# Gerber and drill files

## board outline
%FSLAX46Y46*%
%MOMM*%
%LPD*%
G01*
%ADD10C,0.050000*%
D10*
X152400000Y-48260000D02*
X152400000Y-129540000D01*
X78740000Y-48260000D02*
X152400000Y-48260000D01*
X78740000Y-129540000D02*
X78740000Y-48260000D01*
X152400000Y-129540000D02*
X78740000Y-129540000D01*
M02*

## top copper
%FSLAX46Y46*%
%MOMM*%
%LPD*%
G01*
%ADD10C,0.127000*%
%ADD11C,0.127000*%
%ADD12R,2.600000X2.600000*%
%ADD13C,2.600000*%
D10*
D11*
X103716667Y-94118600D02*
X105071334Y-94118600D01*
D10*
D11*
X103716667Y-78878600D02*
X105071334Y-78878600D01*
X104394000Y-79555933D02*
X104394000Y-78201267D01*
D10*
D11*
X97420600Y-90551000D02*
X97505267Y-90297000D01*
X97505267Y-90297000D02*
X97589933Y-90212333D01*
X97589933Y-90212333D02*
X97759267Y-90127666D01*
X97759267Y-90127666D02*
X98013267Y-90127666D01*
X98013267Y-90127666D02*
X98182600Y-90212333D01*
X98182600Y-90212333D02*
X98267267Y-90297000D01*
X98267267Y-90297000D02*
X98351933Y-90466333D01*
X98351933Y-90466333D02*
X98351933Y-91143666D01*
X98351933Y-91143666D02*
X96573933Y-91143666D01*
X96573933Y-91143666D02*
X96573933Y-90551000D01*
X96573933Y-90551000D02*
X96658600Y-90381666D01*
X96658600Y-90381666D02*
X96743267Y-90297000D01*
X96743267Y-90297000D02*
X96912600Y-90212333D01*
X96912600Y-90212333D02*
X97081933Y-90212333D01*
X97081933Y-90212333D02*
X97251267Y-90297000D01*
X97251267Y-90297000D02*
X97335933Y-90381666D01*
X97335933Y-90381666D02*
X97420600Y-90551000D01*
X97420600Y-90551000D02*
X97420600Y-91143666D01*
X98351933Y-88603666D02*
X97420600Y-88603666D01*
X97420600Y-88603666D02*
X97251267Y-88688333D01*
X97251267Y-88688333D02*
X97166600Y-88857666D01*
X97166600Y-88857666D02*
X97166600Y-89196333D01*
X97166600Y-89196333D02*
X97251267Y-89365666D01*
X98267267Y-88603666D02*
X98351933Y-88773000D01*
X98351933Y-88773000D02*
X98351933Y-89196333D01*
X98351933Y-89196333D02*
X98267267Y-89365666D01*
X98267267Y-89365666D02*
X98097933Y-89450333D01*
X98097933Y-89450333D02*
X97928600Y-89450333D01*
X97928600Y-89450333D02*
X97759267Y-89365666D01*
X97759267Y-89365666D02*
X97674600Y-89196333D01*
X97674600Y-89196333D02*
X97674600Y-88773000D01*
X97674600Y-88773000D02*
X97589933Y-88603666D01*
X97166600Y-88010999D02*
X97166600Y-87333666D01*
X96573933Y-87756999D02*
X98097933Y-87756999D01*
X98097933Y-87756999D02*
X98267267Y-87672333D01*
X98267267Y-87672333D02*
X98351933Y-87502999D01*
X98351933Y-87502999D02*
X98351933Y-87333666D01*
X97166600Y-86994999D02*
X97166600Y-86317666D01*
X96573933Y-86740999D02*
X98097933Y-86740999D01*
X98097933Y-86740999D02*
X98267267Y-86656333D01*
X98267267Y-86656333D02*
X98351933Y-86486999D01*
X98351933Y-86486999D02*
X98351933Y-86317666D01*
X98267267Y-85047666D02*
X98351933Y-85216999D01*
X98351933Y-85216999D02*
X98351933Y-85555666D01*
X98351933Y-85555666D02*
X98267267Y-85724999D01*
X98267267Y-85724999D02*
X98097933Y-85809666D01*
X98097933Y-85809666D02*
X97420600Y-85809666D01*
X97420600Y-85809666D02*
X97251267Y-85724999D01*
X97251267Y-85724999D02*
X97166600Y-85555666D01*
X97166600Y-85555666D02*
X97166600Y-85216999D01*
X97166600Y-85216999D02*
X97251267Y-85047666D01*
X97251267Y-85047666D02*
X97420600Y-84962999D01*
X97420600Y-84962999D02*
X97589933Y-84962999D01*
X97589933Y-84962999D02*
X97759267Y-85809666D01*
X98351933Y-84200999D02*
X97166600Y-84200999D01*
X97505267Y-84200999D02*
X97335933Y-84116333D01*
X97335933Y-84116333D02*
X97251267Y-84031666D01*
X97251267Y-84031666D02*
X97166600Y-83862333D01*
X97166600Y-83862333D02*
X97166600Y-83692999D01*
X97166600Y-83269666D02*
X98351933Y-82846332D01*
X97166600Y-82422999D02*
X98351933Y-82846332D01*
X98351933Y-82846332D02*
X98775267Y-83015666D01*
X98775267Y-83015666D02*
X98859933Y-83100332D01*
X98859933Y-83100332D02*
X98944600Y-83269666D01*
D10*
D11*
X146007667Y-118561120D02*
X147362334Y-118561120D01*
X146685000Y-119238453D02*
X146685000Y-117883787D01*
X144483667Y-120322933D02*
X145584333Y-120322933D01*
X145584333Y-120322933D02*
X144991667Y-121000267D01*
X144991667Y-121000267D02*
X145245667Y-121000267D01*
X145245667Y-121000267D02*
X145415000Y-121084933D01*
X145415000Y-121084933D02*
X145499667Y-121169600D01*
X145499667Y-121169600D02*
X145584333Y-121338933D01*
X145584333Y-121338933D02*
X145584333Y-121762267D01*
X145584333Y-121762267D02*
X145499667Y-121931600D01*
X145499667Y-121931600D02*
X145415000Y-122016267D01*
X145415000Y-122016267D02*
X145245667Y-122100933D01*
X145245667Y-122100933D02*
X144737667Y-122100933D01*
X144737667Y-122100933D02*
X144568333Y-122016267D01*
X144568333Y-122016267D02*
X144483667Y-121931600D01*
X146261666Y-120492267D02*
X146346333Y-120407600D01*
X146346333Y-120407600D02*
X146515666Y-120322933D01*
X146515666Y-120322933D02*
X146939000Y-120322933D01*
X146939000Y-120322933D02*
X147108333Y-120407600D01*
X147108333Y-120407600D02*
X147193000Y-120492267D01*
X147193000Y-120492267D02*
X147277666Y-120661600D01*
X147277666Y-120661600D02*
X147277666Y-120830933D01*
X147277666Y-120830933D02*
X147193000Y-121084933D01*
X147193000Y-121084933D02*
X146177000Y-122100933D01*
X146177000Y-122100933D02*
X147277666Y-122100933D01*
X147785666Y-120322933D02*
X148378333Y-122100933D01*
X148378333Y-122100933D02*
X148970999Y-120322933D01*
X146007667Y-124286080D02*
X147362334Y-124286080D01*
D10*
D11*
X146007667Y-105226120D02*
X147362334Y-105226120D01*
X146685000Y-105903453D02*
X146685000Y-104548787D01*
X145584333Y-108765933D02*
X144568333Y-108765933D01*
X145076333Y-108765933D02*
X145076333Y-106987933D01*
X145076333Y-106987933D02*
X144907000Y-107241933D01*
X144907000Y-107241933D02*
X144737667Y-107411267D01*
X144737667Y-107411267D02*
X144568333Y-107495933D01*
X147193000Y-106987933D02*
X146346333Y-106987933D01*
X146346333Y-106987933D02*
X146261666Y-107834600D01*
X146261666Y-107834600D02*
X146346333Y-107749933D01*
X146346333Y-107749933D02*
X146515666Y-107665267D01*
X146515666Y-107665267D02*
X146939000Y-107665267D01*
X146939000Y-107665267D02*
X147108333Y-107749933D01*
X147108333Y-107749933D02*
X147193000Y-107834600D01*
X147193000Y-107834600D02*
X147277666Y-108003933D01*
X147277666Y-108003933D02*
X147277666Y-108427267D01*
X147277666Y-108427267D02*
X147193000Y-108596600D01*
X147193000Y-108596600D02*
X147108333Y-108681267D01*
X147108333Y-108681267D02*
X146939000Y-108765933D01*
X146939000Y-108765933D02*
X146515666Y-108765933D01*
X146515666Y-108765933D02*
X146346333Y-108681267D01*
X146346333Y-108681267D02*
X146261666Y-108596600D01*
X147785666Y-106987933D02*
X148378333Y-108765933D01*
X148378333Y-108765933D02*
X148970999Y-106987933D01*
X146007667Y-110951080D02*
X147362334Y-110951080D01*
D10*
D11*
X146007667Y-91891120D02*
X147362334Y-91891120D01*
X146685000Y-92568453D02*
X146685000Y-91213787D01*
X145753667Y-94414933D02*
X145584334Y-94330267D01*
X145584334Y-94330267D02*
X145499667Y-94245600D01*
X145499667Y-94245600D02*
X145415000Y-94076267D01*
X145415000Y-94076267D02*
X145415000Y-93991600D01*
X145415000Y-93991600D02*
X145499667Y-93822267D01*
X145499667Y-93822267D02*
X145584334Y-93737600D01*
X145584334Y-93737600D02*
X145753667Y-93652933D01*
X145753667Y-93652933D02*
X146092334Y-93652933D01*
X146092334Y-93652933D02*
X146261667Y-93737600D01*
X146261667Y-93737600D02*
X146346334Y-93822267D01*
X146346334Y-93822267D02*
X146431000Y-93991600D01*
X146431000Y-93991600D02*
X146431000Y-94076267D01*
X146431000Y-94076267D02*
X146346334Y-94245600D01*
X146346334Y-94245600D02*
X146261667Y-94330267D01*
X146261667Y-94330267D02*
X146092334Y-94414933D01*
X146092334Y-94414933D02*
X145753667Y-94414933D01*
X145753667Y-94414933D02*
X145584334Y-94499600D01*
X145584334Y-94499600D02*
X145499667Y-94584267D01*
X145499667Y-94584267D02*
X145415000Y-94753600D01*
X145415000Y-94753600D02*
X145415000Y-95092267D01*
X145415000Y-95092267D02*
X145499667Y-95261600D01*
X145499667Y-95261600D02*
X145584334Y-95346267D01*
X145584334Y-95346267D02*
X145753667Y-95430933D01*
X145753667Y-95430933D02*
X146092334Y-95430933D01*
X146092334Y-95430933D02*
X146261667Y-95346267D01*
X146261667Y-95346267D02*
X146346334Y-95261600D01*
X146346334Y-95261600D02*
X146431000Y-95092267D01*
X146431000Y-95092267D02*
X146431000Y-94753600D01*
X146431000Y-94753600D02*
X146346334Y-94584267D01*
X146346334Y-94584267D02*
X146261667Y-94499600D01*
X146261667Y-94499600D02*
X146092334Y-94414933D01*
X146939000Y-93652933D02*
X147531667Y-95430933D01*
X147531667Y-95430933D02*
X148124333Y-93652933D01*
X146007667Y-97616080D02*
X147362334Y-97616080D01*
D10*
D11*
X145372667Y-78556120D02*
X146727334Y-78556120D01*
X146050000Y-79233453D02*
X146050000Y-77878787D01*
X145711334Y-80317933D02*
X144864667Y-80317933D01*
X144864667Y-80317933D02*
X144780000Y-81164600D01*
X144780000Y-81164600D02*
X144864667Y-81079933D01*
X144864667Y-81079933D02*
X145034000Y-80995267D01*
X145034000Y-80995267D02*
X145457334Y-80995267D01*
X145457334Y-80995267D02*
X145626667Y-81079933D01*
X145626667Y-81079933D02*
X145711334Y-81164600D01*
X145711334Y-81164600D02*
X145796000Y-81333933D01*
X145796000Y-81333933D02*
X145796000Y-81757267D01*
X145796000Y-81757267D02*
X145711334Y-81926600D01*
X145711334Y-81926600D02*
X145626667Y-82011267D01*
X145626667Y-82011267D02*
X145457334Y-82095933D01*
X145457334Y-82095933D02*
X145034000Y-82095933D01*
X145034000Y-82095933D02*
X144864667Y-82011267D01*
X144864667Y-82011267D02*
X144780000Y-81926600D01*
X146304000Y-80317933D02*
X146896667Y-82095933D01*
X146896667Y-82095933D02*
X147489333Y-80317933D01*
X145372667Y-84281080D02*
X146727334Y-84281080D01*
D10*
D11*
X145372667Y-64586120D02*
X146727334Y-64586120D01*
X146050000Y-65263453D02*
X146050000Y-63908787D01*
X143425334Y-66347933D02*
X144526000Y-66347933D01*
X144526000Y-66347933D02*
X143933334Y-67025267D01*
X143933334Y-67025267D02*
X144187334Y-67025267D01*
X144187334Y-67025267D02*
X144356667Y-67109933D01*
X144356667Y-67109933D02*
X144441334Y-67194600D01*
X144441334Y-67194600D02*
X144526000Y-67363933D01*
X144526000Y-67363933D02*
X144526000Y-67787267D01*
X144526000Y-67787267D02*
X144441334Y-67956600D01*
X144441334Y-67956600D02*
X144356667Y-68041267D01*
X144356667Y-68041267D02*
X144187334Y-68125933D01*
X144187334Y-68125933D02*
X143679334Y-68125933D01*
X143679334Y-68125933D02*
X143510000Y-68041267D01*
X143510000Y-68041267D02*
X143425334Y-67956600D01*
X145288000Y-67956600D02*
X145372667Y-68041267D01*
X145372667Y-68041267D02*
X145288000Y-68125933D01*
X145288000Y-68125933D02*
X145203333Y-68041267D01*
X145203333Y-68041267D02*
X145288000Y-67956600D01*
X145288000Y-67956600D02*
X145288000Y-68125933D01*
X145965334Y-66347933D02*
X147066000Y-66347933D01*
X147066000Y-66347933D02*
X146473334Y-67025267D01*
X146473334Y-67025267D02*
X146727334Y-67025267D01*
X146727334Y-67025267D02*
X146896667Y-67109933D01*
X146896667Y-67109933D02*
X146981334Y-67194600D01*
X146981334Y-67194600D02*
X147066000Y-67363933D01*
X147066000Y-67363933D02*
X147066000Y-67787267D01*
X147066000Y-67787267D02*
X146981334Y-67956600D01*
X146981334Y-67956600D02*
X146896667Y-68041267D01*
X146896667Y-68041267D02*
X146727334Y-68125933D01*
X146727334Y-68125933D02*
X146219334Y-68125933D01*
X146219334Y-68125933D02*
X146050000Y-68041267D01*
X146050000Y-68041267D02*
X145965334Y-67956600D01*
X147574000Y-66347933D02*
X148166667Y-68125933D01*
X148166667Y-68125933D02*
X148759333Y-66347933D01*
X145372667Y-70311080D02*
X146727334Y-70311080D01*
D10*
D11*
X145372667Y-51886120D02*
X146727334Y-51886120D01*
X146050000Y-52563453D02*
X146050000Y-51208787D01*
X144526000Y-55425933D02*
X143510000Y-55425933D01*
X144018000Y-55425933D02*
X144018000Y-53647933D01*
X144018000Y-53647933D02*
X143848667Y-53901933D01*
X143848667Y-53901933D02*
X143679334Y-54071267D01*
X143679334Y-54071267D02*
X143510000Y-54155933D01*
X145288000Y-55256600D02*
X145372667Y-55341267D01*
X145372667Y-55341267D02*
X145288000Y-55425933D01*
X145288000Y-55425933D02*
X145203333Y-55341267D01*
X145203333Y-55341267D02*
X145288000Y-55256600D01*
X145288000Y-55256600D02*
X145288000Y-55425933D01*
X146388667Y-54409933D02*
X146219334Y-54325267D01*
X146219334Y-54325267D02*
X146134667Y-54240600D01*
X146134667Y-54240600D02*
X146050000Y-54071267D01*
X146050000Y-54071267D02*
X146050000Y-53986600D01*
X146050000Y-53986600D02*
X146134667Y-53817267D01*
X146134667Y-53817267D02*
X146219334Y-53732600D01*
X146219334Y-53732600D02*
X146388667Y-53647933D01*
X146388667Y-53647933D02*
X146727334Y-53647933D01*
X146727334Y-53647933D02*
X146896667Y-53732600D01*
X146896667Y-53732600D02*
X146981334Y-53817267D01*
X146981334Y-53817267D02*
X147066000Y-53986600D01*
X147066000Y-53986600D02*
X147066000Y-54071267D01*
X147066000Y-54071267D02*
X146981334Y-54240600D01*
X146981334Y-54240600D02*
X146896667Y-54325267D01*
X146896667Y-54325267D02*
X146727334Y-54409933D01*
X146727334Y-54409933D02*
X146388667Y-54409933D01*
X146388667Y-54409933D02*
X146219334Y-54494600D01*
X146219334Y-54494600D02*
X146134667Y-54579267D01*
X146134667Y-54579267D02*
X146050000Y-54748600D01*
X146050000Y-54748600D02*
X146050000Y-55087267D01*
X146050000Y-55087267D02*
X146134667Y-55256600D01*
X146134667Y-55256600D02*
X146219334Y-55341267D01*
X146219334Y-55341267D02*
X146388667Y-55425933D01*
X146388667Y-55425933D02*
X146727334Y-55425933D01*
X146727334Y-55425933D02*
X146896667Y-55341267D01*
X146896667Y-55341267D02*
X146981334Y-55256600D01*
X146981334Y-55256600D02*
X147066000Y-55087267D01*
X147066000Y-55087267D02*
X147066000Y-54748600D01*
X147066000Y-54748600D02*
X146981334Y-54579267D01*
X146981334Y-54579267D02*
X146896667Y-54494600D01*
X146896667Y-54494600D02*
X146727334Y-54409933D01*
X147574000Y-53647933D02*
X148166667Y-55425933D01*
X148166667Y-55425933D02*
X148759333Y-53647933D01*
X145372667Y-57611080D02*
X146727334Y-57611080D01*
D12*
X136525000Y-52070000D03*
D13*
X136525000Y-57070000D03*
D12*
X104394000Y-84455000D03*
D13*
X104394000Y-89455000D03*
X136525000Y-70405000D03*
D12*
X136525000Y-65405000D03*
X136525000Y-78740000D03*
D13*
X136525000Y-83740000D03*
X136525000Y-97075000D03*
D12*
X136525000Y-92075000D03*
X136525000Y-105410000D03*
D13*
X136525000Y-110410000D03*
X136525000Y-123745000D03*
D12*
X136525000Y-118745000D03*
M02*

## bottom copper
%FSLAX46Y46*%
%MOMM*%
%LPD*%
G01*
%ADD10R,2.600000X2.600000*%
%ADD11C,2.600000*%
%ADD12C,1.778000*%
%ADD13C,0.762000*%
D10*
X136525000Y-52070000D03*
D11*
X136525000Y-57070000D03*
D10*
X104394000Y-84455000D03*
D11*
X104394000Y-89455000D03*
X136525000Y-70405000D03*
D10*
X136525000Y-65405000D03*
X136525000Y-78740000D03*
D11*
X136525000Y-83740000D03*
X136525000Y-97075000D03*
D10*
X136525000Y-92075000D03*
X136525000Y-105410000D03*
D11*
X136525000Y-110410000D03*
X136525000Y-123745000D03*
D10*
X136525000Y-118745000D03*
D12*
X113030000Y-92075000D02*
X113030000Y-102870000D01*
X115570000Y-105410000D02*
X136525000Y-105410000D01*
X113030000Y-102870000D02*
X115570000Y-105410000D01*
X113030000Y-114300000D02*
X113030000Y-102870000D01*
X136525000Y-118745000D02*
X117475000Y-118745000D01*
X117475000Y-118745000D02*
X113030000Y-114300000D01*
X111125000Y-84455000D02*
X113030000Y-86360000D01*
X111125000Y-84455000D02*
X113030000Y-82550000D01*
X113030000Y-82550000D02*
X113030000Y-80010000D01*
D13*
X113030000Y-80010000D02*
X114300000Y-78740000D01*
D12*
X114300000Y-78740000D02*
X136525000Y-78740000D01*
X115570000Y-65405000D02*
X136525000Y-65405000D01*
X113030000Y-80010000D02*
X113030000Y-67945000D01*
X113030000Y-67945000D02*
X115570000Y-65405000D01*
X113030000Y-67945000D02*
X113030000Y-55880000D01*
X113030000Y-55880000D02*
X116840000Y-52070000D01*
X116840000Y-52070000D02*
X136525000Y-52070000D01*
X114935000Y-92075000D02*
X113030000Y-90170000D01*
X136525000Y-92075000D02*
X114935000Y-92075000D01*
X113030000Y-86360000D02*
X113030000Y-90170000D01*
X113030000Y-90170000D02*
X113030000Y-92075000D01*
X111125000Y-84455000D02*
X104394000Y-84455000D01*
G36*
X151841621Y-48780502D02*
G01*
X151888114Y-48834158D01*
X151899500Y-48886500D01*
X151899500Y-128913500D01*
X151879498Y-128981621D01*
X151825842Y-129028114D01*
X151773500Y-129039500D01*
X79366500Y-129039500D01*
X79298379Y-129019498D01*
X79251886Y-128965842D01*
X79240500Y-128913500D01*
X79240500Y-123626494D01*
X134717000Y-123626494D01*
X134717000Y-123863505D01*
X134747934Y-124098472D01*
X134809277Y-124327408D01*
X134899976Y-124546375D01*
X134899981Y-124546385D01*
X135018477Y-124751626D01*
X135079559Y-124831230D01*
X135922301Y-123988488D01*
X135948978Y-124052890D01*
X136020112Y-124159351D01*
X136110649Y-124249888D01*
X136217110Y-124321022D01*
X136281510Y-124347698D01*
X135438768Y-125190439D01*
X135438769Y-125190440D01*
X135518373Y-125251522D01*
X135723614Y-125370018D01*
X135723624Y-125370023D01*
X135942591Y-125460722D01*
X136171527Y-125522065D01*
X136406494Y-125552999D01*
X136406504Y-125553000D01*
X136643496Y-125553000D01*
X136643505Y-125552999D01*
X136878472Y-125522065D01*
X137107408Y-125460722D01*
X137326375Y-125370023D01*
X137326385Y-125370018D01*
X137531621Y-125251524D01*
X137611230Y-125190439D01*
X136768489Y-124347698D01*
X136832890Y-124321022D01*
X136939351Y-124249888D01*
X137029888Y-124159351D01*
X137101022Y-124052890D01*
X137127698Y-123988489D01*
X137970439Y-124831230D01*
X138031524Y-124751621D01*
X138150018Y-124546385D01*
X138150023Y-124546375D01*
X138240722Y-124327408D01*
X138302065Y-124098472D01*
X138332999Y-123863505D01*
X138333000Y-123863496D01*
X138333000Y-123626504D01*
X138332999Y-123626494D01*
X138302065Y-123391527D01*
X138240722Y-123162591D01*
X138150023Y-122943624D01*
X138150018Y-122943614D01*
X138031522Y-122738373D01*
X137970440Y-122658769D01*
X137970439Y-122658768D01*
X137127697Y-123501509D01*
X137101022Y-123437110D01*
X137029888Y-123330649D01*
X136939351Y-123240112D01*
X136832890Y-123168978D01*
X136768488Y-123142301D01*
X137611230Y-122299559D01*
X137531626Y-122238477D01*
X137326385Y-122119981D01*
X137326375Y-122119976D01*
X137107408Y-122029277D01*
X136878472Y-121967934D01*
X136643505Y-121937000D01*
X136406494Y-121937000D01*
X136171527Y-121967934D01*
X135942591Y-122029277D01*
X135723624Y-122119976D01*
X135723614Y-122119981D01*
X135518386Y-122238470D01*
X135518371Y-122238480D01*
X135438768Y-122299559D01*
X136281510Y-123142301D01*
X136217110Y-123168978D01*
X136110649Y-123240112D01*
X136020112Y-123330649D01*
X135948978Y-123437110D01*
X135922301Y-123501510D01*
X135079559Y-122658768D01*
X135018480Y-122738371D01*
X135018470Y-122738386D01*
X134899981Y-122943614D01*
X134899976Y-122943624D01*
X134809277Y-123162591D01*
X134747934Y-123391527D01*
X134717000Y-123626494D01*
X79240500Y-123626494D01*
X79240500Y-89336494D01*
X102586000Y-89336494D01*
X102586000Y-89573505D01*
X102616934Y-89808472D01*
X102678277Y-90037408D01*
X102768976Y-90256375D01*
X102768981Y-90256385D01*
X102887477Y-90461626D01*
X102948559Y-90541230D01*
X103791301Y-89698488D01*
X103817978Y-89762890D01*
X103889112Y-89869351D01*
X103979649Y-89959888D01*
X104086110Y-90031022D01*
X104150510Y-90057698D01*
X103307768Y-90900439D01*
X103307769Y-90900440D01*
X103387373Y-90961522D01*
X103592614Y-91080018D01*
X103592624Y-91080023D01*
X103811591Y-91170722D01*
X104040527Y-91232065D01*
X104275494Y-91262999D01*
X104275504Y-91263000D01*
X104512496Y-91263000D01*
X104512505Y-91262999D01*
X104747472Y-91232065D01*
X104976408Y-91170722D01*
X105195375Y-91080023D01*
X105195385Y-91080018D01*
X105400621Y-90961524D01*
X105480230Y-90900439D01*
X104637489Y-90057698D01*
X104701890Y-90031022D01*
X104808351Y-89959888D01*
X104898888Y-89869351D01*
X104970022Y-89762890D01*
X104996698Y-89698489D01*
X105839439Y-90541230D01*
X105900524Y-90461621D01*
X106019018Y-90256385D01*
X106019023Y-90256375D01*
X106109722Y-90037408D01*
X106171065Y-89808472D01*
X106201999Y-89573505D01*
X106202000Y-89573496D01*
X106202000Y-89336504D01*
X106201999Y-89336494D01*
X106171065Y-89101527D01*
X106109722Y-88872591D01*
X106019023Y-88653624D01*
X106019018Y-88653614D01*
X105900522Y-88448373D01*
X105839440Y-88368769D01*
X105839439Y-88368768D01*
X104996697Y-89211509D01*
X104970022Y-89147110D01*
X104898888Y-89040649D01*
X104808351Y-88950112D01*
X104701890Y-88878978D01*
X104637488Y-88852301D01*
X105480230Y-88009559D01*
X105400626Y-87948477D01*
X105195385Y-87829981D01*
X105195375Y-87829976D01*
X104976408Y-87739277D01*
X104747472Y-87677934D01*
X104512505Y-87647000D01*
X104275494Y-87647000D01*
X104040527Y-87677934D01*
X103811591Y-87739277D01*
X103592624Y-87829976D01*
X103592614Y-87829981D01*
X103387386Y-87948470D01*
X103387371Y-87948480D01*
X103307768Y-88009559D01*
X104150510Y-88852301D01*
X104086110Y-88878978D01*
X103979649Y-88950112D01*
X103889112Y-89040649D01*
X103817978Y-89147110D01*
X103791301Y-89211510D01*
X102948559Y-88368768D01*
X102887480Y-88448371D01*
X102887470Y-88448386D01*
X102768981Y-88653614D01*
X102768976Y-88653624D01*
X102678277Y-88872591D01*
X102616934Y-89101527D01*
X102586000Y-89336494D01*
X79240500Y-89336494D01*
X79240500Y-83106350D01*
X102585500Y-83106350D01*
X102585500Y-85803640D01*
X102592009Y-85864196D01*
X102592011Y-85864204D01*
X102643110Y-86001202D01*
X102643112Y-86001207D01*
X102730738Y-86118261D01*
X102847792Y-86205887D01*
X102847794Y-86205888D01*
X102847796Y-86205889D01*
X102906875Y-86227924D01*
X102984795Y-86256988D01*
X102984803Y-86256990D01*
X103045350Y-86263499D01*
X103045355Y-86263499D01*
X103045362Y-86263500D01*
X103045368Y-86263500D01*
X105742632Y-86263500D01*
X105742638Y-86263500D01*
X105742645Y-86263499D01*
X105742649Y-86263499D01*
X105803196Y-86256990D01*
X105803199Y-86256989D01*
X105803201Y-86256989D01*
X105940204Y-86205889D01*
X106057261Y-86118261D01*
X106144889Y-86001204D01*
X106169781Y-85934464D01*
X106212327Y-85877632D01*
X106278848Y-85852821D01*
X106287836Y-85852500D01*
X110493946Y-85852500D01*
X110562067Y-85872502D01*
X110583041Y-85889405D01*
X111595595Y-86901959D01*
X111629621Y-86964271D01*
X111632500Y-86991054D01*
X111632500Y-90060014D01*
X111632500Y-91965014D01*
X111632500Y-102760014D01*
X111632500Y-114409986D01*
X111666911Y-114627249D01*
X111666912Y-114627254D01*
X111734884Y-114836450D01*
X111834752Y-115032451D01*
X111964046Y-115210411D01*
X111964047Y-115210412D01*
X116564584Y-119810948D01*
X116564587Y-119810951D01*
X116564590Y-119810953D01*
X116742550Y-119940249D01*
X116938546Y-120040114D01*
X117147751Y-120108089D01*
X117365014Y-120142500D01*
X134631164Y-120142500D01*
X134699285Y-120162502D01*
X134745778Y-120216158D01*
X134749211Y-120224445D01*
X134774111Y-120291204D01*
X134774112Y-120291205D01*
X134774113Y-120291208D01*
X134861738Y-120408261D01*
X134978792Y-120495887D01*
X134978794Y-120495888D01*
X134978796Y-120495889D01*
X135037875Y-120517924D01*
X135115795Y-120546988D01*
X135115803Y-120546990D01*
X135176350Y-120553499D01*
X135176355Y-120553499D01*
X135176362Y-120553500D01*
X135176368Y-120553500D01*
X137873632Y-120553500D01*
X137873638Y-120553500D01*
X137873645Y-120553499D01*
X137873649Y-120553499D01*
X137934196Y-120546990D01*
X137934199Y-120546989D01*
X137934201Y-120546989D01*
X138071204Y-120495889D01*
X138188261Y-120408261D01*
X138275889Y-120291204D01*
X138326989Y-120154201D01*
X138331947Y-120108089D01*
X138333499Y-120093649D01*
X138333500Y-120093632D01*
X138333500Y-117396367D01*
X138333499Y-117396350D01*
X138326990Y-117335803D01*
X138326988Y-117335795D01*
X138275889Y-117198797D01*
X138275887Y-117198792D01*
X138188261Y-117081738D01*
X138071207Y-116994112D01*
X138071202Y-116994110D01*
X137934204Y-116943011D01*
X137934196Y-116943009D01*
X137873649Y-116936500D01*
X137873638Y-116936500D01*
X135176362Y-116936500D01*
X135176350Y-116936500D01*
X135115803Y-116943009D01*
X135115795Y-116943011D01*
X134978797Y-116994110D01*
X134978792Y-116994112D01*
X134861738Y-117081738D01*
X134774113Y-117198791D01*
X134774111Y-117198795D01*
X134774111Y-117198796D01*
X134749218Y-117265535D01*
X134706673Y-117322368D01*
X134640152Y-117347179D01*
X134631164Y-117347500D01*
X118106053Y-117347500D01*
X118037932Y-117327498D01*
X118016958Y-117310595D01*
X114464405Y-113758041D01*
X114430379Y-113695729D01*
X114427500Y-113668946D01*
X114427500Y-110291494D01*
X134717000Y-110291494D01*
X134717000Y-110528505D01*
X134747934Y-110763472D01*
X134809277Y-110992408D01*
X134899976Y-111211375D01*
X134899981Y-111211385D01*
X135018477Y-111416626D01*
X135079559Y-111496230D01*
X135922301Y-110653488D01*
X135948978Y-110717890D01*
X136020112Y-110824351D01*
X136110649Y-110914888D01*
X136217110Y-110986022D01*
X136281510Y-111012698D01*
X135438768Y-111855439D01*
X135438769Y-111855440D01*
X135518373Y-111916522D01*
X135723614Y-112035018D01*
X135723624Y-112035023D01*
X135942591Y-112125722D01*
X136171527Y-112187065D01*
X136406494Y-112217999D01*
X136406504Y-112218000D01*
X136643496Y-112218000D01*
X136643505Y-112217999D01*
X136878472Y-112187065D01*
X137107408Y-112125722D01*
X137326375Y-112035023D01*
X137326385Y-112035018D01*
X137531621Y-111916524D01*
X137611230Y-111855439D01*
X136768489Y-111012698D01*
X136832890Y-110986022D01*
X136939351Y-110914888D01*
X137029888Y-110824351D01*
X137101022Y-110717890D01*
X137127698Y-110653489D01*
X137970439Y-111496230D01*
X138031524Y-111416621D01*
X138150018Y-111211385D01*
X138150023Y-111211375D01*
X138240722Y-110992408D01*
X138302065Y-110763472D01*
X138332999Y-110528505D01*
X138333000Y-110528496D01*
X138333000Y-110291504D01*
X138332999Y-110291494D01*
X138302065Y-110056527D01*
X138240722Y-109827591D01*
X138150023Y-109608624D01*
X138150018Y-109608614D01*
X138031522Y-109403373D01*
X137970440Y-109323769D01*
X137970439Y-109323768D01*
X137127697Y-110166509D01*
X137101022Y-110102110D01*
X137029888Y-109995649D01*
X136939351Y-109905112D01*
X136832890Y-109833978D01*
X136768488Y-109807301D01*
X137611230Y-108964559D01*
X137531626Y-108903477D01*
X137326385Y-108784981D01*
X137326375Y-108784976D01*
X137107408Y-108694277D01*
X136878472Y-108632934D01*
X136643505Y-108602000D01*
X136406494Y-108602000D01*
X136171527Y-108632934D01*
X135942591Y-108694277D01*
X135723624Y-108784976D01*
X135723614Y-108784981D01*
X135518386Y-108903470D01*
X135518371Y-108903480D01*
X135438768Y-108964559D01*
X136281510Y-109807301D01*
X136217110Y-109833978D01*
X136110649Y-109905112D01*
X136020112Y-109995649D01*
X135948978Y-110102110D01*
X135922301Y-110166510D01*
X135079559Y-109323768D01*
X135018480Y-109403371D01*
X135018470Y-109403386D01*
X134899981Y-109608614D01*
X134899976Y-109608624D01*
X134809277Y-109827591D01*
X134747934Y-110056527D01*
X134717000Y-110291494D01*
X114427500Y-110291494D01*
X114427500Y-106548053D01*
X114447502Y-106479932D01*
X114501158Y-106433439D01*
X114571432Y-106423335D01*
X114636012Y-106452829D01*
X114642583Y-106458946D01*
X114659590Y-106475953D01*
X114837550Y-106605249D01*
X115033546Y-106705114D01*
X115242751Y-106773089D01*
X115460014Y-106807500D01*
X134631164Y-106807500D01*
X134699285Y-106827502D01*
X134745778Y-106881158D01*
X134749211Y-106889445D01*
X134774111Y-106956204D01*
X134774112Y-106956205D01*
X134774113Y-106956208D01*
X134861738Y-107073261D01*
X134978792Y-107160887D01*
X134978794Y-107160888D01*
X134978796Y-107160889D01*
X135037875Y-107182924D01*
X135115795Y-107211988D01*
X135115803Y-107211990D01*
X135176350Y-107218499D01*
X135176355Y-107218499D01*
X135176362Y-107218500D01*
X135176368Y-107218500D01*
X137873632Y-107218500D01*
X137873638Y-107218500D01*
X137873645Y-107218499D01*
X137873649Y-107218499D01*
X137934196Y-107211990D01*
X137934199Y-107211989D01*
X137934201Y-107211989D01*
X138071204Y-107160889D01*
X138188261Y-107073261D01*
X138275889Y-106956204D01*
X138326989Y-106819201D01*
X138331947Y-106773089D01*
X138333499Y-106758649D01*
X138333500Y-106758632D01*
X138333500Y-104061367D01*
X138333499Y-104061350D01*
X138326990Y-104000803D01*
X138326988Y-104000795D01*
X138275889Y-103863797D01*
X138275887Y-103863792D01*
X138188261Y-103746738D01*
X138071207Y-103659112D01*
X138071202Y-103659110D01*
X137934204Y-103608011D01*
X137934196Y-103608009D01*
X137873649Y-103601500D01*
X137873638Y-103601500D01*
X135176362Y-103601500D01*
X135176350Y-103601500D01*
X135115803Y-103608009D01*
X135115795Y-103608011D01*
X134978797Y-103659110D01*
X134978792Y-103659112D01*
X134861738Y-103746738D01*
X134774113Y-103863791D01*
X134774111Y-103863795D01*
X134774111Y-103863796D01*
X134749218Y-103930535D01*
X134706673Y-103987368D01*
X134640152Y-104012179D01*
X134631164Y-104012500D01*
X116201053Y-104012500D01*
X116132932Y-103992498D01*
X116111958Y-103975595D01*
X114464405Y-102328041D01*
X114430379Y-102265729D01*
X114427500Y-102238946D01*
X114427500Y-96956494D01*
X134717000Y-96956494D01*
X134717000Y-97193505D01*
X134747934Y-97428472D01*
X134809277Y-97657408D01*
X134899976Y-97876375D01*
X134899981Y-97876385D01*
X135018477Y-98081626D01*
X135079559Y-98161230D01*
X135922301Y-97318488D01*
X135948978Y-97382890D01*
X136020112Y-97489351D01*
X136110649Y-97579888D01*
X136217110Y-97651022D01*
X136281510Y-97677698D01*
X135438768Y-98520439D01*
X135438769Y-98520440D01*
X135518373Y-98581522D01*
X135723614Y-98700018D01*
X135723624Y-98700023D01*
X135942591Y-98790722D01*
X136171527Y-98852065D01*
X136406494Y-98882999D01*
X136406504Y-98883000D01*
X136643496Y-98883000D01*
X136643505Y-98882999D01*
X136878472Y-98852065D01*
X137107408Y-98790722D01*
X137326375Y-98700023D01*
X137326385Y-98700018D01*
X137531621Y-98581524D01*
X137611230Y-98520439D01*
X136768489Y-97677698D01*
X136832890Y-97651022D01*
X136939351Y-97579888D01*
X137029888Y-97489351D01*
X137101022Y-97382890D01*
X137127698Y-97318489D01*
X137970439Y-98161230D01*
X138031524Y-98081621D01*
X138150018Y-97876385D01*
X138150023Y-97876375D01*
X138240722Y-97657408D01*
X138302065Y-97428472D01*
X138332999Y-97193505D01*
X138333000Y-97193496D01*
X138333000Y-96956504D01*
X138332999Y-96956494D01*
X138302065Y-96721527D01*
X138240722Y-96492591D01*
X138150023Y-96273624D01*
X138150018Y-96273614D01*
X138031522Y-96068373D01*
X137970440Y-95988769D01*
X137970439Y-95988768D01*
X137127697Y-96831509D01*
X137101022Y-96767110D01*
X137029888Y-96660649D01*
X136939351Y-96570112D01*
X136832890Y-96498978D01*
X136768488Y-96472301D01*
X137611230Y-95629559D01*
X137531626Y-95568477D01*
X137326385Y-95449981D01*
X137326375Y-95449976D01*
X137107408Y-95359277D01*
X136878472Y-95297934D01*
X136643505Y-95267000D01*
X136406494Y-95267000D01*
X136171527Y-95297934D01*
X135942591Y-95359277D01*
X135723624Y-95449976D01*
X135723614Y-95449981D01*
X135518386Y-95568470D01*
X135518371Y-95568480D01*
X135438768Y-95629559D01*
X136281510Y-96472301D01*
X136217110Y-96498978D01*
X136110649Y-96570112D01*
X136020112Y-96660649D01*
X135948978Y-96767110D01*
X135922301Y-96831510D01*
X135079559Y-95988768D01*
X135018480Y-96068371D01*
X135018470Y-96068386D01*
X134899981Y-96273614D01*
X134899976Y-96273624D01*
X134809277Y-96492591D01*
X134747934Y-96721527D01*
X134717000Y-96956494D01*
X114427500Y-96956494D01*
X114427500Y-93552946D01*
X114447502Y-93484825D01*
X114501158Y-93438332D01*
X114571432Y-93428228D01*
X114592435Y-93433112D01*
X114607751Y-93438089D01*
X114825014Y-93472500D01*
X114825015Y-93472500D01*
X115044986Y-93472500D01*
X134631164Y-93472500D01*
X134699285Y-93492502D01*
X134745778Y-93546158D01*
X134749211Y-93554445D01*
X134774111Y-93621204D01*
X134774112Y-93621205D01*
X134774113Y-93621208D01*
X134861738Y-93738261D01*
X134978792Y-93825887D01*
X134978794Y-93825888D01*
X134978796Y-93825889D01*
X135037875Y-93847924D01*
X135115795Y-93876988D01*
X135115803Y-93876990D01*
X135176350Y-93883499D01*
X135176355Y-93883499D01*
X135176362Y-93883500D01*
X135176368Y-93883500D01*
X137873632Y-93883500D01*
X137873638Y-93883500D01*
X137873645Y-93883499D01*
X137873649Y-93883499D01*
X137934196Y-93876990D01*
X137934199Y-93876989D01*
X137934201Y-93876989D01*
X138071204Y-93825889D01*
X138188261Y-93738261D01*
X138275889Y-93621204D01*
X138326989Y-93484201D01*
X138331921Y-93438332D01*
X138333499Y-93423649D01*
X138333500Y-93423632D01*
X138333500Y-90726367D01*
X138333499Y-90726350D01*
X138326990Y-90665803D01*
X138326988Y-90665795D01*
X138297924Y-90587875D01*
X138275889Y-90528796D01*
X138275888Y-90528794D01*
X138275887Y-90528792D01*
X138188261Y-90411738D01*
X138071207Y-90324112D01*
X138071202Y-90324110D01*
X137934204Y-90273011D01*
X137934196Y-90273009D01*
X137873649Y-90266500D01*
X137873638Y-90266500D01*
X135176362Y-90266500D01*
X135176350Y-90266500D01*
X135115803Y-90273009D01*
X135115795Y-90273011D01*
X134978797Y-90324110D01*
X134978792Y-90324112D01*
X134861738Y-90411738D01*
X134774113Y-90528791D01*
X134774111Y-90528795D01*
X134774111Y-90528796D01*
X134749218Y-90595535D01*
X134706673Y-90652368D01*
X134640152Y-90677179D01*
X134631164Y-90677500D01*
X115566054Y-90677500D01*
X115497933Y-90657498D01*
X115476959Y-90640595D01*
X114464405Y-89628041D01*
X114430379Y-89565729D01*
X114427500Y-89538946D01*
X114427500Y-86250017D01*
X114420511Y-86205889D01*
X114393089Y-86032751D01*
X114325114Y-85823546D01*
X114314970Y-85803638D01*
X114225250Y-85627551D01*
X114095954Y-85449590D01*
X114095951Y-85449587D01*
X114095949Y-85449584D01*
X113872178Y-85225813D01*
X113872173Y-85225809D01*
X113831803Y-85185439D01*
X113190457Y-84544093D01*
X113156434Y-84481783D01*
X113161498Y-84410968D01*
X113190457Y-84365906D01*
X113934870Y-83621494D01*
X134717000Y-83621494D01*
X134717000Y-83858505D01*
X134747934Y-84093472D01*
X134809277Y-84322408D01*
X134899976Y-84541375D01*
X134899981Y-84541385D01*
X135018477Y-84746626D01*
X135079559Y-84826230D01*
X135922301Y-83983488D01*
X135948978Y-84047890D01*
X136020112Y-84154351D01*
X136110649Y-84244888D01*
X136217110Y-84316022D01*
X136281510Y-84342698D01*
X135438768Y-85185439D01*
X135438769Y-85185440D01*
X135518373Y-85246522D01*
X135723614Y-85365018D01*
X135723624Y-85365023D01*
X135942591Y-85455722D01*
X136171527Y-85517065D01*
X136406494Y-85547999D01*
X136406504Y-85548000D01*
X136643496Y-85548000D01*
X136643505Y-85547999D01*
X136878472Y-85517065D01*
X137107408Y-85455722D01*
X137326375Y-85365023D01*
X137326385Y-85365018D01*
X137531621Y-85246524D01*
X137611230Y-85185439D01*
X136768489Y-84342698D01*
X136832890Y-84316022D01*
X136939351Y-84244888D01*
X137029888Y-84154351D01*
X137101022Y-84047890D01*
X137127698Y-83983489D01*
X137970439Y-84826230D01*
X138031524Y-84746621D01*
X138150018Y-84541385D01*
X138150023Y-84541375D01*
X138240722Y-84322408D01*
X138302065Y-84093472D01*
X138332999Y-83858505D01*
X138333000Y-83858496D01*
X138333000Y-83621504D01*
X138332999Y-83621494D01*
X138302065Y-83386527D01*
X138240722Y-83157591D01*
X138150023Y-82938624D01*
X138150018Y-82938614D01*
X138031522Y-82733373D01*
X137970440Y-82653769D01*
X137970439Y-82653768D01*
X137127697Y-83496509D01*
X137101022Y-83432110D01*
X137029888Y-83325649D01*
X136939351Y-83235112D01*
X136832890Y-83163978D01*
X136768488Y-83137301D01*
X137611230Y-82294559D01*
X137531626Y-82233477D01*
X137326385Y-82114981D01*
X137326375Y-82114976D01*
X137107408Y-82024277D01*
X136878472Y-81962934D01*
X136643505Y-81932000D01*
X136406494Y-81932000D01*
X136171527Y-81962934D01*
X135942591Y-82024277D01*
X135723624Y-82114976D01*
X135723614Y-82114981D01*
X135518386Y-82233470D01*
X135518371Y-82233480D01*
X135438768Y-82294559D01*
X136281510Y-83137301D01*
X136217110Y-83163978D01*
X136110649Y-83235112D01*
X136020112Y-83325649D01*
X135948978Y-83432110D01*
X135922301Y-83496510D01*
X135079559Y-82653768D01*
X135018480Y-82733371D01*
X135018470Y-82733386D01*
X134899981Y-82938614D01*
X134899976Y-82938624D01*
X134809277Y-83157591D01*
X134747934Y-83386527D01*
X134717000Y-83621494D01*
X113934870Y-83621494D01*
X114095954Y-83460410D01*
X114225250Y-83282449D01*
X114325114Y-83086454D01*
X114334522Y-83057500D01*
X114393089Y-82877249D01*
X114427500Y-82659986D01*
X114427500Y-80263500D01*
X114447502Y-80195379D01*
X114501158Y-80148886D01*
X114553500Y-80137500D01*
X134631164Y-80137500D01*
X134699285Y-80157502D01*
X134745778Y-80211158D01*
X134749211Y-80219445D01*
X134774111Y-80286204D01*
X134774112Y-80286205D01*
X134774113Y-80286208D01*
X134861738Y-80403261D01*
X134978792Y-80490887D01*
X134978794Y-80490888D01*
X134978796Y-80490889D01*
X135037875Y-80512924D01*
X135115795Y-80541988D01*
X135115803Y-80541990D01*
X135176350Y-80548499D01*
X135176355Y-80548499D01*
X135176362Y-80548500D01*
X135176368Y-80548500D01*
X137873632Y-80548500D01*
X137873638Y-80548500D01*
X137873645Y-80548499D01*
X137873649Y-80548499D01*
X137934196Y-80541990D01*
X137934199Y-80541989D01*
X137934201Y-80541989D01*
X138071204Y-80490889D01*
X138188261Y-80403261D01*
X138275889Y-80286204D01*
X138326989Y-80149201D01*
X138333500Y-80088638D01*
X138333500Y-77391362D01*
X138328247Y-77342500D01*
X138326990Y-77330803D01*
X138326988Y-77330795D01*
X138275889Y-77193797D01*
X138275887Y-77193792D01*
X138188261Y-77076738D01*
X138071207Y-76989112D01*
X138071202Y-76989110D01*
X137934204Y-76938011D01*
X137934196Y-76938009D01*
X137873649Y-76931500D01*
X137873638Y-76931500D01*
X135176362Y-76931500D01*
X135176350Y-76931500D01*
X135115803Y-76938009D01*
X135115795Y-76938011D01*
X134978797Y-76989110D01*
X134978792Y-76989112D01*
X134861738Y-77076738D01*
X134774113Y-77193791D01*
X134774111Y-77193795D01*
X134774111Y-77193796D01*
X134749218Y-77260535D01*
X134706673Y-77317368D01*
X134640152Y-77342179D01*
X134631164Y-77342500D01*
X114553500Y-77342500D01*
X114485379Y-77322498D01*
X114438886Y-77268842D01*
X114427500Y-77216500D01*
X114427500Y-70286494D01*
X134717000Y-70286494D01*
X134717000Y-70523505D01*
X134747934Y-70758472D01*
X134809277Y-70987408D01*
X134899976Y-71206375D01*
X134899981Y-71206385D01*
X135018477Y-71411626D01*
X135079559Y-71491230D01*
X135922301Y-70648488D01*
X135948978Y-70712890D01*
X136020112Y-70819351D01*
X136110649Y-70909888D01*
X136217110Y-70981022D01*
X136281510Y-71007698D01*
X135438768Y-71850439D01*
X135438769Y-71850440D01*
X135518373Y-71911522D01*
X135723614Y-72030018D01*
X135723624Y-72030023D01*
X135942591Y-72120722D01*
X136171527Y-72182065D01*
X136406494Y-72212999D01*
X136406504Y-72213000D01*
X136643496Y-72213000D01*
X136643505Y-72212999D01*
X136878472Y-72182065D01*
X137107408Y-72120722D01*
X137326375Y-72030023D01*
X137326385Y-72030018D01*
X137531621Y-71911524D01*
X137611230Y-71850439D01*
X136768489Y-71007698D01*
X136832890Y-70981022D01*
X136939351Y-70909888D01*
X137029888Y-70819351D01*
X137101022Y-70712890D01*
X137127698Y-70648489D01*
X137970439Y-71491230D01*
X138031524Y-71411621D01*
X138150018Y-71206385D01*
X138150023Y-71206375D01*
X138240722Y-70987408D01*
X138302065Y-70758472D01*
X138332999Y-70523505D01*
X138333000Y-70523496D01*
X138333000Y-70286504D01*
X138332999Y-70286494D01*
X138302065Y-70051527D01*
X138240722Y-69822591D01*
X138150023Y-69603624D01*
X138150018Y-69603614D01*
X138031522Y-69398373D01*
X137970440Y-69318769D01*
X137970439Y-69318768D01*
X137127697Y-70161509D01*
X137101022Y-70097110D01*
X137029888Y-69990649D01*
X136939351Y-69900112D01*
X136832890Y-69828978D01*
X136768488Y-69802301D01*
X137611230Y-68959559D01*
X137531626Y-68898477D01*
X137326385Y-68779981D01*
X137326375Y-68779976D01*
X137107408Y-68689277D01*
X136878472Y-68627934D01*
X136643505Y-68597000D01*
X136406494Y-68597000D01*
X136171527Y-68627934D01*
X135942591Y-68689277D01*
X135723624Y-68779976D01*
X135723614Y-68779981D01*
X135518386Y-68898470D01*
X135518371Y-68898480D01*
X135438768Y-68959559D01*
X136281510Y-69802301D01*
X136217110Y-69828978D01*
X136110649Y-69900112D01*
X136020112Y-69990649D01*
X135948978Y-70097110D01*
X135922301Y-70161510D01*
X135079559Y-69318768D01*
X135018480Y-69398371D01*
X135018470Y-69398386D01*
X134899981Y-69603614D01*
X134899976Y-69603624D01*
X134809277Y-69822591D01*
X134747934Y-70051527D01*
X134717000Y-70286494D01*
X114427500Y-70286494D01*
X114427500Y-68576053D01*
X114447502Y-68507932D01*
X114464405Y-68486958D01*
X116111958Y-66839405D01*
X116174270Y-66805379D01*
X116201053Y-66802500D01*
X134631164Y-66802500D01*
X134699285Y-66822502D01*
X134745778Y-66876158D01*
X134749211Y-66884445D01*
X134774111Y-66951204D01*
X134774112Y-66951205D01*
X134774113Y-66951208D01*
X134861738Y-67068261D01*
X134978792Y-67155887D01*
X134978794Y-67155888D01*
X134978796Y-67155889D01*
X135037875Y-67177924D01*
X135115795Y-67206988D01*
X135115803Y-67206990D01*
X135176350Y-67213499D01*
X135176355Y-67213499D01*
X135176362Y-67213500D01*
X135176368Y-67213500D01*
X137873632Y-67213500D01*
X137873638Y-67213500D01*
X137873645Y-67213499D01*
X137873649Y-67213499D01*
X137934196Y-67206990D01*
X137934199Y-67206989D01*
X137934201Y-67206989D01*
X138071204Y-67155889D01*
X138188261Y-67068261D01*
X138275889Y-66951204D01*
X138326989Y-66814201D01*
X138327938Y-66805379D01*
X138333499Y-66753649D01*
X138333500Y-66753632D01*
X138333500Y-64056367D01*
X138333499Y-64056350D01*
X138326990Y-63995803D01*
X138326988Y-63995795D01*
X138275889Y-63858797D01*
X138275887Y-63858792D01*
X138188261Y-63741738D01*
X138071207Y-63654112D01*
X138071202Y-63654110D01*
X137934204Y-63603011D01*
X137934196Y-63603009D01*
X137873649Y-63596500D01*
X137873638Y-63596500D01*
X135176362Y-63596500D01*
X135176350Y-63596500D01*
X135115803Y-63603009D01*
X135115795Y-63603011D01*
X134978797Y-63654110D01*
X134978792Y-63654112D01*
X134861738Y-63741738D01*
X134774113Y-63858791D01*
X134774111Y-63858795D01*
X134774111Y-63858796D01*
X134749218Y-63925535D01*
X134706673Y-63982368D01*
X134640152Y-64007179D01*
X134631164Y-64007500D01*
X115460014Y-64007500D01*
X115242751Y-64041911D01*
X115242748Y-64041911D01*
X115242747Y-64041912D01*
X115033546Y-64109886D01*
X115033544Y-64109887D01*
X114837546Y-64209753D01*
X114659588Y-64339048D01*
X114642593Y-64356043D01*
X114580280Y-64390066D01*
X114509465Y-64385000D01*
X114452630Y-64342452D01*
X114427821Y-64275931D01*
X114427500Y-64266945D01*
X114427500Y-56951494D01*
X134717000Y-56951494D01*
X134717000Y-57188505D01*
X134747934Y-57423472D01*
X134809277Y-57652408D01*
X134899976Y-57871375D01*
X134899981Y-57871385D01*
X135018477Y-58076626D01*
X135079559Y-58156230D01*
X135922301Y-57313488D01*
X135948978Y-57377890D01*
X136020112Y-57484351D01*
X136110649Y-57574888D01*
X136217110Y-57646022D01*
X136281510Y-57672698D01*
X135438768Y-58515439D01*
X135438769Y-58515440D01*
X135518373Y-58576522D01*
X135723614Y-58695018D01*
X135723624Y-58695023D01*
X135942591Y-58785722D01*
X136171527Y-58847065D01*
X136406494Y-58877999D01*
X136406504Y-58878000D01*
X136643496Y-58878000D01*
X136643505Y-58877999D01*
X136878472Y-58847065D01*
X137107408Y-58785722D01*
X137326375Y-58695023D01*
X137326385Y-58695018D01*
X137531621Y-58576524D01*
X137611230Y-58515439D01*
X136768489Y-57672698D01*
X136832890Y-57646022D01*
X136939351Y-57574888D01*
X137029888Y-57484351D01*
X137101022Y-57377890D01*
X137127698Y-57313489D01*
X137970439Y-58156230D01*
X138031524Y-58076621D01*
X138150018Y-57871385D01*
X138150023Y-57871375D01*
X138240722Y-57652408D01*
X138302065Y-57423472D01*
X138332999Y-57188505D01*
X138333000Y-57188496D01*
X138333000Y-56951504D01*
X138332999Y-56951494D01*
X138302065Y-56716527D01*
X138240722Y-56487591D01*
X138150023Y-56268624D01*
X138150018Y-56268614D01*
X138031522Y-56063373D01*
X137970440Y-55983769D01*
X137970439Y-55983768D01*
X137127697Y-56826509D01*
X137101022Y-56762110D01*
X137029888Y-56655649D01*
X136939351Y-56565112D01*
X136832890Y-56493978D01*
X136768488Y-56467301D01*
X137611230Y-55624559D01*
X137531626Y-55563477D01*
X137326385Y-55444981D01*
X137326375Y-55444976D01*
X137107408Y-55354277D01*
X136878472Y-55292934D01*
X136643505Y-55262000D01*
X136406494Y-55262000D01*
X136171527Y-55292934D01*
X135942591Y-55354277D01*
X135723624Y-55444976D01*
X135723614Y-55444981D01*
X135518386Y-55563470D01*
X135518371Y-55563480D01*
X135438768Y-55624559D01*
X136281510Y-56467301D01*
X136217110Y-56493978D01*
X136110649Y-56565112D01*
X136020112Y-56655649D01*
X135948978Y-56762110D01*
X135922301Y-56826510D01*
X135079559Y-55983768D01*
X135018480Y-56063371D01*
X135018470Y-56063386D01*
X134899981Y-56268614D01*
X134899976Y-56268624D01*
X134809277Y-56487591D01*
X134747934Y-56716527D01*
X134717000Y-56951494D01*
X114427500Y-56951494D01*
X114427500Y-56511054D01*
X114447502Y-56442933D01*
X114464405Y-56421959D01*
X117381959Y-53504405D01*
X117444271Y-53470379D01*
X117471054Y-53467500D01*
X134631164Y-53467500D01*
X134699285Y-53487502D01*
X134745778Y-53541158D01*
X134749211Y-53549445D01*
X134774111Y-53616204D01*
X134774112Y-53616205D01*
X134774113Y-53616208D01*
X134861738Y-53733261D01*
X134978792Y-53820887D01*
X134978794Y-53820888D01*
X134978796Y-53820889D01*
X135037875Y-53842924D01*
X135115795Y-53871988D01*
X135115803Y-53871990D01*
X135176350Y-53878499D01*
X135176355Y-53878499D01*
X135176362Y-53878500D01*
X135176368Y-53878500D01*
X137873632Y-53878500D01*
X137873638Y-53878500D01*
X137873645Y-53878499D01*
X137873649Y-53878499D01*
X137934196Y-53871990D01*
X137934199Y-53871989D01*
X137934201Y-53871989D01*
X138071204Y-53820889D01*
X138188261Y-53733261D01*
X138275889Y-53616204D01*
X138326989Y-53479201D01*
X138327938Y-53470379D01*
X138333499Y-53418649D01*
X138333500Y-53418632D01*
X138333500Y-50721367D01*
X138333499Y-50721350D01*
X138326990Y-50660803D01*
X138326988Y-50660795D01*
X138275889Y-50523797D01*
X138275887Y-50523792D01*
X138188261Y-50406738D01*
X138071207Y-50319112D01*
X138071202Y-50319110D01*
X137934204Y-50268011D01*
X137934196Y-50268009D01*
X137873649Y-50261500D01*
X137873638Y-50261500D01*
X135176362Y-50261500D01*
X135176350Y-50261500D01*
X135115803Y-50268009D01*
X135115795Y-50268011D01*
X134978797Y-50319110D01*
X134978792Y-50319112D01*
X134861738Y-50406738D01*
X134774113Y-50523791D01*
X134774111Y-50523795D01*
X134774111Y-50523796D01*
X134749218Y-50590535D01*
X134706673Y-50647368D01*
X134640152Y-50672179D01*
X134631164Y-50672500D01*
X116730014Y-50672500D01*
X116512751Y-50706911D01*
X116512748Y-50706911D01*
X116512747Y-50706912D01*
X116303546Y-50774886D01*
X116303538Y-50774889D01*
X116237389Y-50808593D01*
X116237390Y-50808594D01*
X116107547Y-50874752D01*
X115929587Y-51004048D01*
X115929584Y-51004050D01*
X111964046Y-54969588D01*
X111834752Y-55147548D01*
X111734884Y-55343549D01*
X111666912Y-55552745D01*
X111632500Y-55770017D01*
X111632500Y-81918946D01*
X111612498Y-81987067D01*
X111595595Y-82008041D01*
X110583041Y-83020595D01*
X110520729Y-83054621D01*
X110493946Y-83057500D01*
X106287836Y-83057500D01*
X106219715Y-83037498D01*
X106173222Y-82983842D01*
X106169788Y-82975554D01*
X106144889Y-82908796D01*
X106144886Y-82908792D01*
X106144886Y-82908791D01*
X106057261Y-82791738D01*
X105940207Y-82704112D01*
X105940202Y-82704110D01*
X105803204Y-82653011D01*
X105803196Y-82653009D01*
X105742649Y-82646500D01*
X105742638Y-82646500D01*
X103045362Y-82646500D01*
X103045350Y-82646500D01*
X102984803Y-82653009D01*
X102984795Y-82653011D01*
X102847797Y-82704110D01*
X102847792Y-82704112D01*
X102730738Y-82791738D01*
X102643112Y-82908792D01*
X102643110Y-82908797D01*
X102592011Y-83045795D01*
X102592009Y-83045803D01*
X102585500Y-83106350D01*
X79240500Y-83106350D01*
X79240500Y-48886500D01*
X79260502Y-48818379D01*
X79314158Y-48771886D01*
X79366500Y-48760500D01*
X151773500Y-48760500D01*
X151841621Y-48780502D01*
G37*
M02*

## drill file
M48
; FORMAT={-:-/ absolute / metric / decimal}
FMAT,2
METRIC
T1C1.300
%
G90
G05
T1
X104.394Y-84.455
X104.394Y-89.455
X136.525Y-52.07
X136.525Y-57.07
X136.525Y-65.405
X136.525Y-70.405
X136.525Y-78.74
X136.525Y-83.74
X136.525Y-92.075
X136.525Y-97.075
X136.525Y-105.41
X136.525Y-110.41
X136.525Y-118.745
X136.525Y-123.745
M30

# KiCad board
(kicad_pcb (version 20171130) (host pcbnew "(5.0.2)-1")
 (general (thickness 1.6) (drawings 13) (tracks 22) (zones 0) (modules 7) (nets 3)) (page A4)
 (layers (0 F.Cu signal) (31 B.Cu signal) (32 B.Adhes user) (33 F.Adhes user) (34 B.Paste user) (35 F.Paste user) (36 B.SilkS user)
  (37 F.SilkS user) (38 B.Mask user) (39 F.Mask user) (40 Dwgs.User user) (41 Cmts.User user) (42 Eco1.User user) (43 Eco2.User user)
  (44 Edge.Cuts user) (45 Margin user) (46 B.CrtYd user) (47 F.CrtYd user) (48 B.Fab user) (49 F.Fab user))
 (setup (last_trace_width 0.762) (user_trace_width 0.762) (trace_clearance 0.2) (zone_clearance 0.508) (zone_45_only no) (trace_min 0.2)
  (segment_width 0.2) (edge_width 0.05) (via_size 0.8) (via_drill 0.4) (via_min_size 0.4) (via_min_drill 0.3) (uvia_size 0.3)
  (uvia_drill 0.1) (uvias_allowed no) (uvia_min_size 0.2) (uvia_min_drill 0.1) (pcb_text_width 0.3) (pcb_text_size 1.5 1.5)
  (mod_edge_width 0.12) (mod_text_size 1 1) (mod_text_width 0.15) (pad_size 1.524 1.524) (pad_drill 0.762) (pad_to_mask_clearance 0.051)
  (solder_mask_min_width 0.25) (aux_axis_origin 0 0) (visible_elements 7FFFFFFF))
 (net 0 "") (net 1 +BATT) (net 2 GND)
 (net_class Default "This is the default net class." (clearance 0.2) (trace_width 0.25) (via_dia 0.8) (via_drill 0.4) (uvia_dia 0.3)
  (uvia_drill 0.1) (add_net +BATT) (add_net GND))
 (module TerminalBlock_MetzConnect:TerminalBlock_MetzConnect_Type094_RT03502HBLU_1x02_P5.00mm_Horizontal (layer F.Cu) (at 136.525 52.07 270)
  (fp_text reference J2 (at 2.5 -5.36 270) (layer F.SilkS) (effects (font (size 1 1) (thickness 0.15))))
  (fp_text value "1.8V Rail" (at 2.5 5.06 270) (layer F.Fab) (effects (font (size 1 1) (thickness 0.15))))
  (pad 1 thru_hole rect (at 0 0 270) (size 2.6 2.6) (drill 1.3) (layers *.Cu *.Mask) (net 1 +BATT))
  (pad 2 thru_hole circle (at 5 0 270) (size 2.6 2.6) (drill 1.3) (layers *.Cu *.Mask) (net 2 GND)))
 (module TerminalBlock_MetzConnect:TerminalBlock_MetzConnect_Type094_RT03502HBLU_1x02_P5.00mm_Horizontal (layer F.Cu)
  (at 104.394 84.455 270)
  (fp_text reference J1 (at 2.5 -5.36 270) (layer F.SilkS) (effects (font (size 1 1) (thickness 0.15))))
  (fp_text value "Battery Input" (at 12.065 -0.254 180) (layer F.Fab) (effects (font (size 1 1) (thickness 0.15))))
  (pad 1 thru_hole rect (at 0 0 270) (size 2.6 2.6) (drill 1.3) (layers *.Cu *.Mask) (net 1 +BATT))
  (pad 2 thru_hole circle (at 5 0 270) (size 2.6 2.6) (drill 1.3) (layers *.Cu *.Mask) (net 2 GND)))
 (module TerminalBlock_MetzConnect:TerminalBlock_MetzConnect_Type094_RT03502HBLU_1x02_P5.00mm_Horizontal (layer F.Cu)
  (at 136.525 65.405 270)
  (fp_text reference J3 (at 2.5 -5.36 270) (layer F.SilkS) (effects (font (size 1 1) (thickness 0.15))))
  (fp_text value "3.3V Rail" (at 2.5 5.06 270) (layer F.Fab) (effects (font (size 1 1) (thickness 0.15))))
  (pad 2 thru_hole circle (at 5 0 270) (size 2.6 2.6) (drill 1.3) (layers *.Cu *.Mask) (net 2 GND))
  (pad 1 thru_hole rect (at 0 0 270) (size 2.6 2.6) (drill 1.3) (layers *.Cu *.Mask) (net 1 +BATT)))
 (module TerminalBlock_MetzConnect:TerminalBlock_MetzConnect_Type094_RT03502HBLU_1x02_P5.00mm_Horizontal (layer F.Cu) (at 136.525 78.74 270)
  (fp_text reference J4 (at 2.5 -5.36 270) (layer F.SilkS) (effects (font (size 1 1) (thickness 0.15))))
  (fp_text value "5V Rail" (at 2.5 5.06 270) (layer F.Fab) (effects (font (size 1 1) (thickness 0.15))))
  (pad 1 thru_hole rect (at 0 0 270) (size 2.6 2.6) (drill 1.3) (layers *.Cu *.Mask) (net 1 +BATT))
  (pad 2 thru_hole circle (at 5 0 270) (size 2.6 2.6) (drill 1.3) (layers *.Cu *.Mask) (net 2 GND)))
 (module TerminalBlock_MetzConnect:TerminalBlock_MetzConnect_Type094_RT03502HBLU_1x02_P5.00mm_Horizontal (layer F.Cu)
  (at 136.525 92.075 270)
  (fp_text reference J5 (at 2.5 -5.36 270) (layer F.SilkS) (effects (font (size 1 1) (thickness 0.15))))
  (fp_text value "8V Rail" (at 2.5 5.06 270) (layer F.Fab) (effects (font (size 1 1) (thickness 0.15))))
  (pad 2 thru_hole circle (at 5 0 270) (size 2.6 2.6) (drill 1.3) (layers *.Cu *.Mask) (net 2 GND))
  (pad 1 thru_hole rect (at 0 0 270) (size 2.6 2.6) (drill 1.3) (layers *.Cu *.Mask) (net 1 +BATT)))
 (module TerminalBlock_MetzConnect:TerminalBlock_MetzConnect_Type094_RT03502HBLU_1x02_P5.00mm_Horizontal (layer F.Cu)
  (at 136.525 105.41 270)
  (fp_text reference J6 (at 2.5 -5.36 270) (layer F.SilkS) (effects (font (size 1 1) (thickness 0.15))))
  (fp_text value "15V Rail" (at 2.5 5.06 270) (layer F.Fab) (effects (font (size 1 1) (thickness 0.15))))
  (pad 1 thru_hole rect (at 0 0 270) (size 2.6 2.6) (drill 1.3) (layers *.Cu *.Mask) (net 1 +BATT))
  (pad 2 thru_hole circle (at 5 0 270) (size 2.6 2.6) (drill 1.3) (layers *.Cu *.Mask) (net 2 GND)))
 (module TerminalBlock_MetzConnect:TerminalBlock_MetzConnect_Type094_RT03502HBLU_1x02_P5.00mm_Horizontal (layer F.Cu)
  (at 136.525 118.745 270)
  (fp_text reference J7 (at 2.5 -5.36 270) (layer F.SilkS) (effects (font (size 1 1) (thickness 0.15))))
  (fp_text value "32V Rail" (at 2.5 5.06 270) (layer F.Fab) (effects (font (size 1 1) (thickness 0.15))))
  (pad 2 thru_hole circle (at 5 0 270) (size 2.6 2.6) (drill 1.3) (layers *.Cu *.Mask) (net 2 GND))
  (pad 1 thru_hole rect (at 0 0 270) (size 2.6 2.6) (drill 1.3) (layers *.Cu *.Mask) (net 1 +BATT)))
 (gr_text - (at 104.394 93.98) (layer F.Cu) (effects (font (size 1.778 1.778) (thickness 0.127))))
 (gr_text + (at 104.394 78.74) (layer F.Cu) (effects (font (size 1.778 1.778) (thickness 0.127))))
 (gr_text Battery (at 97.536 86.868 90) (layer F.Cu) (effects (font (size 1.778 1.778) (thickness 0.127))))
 (gr_line (start 152.4 48.26) (end 152.4 129.54) (layer Edge.Cuts) (width 0.05))
 (gr_line (start 78.74 48.26) (end 152.4 48.26) (layer Edge.Cuts) (width 0.05))
 (gr_line (start 78.74 129.54) (end 78.74 48.26) (layer Edge.Cuts) (width 0.05))
 (gr_line (start 152.4 129.54) (end 78.74 129.54) (layer Edge.Cuts) (width 0.05))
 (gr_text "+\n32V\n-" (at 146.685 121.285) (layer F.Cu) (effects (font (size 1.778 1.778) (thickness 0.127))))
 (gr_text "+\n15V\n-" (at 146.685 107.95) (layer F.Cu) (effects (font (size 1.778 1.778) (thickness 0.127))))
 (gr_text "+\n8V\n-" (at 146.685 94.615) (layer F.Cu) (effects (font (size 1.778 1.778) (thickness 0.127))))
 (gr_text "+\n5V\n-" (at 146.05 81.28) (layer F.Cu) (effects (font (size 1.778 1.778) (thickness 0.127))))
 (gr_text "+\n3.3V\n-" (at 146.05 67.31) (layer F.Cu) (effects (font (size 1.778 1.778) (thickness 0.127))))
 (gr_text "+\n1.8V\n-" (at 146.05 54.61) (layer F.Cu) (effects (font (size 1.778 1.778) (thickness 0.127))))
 (segment (start 113.03 92.075) (end 113.03 102.87) (width 1.778) (layer B.Cu) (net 1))
 (segment (start 115.57 105.41) (end 136.525 105.41) (width 1.778) (layer B.Cu) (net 1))
 (segment (start 113.03 102.87) (end 115.57 105.41) (width 1.778) (layer B.Cu) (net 1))
 (segment (start 113.03 114.3) (end 113.03 102.87) (width 1.778) (layer B.Cu) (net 1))
 (segment (start 136.525 118.745) (end 117.475 118.745) (width 1.778) (layer B.Cu) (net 1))
 (segment (start 117.475 118.745) (end 113.03 114.3) (width 1.778) (layer B.Cu) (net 1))
 (segment (start 111.125 84.455) (end 113.03 86.36) (width 1.778) (layer B.Cu) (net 1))
 (segment (start 111.125 84.455) (end 113.03 82.55) (width 1.778) (layer B.Cu) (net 1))
 (segment (start 113.03 82.55) (end 113.03 80.01) (width 1.778) (layer B.Cu) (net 1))
 (segment (start 113.03 80.01) (end 114.3 78.74) (width 0.762) (layer B.Cu) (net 1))
 (segment (start 114.3 78.74) (end 136.525 78.74) (width 1.778) (layer B.Cu) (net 1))
 (segment (start 115.57 65.405) (end 136.525 65.405) (width 1.778) (layer B.Cu) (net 1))
 (segment (start 113.03 80.01) (end 113.03 67.945) (width 1.778) (layer B.Cu) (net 1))
 (segment (start 113.03 67.945) (end 115.57 65.405) (width 1.778) (layer B.Cu) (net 1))
 (segment (start 113.03 67.945) (end 113.03 55.88) (width 1.778) (layer B.Cu) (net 1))
 (segment (start 113.03 55.88) (end 116.84 52.07) (width 1.778) (layer B.Cu) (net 1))
 (segment (start 116.84 52.07) (end 136.525 52.07) (width 1.778) (layer B.Cu) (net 1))
 (segment (start 114.935 92.075) (end 113.03 90.17) (width 1.778) (layer B.Cu) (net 1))
 (segment (start 136.525 92.075) (end 114.935 92.075) (width 1.778) (layer B.Cu) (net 1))
 (segment (start 113.03 86.36) (end 113.03 90.17) (width 1.778) (layer B.Cu) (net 1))
 (segment (start 113.03 90.17) (end 113.03 92.075) (width 1.778) (layer B.Cu) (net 1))
 (segment (start 111.125 84.455) (end 104.394 84.455) (width 1.778) (layer B.Cu) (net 1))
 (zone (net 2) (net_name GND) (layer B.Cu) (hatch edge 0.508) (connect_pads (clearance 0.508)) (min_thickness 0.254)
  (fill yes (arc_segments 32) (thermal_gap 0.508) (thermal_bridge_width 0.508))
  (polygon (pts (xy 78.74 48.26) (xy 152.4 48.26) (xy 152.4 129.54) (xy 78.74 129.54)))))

